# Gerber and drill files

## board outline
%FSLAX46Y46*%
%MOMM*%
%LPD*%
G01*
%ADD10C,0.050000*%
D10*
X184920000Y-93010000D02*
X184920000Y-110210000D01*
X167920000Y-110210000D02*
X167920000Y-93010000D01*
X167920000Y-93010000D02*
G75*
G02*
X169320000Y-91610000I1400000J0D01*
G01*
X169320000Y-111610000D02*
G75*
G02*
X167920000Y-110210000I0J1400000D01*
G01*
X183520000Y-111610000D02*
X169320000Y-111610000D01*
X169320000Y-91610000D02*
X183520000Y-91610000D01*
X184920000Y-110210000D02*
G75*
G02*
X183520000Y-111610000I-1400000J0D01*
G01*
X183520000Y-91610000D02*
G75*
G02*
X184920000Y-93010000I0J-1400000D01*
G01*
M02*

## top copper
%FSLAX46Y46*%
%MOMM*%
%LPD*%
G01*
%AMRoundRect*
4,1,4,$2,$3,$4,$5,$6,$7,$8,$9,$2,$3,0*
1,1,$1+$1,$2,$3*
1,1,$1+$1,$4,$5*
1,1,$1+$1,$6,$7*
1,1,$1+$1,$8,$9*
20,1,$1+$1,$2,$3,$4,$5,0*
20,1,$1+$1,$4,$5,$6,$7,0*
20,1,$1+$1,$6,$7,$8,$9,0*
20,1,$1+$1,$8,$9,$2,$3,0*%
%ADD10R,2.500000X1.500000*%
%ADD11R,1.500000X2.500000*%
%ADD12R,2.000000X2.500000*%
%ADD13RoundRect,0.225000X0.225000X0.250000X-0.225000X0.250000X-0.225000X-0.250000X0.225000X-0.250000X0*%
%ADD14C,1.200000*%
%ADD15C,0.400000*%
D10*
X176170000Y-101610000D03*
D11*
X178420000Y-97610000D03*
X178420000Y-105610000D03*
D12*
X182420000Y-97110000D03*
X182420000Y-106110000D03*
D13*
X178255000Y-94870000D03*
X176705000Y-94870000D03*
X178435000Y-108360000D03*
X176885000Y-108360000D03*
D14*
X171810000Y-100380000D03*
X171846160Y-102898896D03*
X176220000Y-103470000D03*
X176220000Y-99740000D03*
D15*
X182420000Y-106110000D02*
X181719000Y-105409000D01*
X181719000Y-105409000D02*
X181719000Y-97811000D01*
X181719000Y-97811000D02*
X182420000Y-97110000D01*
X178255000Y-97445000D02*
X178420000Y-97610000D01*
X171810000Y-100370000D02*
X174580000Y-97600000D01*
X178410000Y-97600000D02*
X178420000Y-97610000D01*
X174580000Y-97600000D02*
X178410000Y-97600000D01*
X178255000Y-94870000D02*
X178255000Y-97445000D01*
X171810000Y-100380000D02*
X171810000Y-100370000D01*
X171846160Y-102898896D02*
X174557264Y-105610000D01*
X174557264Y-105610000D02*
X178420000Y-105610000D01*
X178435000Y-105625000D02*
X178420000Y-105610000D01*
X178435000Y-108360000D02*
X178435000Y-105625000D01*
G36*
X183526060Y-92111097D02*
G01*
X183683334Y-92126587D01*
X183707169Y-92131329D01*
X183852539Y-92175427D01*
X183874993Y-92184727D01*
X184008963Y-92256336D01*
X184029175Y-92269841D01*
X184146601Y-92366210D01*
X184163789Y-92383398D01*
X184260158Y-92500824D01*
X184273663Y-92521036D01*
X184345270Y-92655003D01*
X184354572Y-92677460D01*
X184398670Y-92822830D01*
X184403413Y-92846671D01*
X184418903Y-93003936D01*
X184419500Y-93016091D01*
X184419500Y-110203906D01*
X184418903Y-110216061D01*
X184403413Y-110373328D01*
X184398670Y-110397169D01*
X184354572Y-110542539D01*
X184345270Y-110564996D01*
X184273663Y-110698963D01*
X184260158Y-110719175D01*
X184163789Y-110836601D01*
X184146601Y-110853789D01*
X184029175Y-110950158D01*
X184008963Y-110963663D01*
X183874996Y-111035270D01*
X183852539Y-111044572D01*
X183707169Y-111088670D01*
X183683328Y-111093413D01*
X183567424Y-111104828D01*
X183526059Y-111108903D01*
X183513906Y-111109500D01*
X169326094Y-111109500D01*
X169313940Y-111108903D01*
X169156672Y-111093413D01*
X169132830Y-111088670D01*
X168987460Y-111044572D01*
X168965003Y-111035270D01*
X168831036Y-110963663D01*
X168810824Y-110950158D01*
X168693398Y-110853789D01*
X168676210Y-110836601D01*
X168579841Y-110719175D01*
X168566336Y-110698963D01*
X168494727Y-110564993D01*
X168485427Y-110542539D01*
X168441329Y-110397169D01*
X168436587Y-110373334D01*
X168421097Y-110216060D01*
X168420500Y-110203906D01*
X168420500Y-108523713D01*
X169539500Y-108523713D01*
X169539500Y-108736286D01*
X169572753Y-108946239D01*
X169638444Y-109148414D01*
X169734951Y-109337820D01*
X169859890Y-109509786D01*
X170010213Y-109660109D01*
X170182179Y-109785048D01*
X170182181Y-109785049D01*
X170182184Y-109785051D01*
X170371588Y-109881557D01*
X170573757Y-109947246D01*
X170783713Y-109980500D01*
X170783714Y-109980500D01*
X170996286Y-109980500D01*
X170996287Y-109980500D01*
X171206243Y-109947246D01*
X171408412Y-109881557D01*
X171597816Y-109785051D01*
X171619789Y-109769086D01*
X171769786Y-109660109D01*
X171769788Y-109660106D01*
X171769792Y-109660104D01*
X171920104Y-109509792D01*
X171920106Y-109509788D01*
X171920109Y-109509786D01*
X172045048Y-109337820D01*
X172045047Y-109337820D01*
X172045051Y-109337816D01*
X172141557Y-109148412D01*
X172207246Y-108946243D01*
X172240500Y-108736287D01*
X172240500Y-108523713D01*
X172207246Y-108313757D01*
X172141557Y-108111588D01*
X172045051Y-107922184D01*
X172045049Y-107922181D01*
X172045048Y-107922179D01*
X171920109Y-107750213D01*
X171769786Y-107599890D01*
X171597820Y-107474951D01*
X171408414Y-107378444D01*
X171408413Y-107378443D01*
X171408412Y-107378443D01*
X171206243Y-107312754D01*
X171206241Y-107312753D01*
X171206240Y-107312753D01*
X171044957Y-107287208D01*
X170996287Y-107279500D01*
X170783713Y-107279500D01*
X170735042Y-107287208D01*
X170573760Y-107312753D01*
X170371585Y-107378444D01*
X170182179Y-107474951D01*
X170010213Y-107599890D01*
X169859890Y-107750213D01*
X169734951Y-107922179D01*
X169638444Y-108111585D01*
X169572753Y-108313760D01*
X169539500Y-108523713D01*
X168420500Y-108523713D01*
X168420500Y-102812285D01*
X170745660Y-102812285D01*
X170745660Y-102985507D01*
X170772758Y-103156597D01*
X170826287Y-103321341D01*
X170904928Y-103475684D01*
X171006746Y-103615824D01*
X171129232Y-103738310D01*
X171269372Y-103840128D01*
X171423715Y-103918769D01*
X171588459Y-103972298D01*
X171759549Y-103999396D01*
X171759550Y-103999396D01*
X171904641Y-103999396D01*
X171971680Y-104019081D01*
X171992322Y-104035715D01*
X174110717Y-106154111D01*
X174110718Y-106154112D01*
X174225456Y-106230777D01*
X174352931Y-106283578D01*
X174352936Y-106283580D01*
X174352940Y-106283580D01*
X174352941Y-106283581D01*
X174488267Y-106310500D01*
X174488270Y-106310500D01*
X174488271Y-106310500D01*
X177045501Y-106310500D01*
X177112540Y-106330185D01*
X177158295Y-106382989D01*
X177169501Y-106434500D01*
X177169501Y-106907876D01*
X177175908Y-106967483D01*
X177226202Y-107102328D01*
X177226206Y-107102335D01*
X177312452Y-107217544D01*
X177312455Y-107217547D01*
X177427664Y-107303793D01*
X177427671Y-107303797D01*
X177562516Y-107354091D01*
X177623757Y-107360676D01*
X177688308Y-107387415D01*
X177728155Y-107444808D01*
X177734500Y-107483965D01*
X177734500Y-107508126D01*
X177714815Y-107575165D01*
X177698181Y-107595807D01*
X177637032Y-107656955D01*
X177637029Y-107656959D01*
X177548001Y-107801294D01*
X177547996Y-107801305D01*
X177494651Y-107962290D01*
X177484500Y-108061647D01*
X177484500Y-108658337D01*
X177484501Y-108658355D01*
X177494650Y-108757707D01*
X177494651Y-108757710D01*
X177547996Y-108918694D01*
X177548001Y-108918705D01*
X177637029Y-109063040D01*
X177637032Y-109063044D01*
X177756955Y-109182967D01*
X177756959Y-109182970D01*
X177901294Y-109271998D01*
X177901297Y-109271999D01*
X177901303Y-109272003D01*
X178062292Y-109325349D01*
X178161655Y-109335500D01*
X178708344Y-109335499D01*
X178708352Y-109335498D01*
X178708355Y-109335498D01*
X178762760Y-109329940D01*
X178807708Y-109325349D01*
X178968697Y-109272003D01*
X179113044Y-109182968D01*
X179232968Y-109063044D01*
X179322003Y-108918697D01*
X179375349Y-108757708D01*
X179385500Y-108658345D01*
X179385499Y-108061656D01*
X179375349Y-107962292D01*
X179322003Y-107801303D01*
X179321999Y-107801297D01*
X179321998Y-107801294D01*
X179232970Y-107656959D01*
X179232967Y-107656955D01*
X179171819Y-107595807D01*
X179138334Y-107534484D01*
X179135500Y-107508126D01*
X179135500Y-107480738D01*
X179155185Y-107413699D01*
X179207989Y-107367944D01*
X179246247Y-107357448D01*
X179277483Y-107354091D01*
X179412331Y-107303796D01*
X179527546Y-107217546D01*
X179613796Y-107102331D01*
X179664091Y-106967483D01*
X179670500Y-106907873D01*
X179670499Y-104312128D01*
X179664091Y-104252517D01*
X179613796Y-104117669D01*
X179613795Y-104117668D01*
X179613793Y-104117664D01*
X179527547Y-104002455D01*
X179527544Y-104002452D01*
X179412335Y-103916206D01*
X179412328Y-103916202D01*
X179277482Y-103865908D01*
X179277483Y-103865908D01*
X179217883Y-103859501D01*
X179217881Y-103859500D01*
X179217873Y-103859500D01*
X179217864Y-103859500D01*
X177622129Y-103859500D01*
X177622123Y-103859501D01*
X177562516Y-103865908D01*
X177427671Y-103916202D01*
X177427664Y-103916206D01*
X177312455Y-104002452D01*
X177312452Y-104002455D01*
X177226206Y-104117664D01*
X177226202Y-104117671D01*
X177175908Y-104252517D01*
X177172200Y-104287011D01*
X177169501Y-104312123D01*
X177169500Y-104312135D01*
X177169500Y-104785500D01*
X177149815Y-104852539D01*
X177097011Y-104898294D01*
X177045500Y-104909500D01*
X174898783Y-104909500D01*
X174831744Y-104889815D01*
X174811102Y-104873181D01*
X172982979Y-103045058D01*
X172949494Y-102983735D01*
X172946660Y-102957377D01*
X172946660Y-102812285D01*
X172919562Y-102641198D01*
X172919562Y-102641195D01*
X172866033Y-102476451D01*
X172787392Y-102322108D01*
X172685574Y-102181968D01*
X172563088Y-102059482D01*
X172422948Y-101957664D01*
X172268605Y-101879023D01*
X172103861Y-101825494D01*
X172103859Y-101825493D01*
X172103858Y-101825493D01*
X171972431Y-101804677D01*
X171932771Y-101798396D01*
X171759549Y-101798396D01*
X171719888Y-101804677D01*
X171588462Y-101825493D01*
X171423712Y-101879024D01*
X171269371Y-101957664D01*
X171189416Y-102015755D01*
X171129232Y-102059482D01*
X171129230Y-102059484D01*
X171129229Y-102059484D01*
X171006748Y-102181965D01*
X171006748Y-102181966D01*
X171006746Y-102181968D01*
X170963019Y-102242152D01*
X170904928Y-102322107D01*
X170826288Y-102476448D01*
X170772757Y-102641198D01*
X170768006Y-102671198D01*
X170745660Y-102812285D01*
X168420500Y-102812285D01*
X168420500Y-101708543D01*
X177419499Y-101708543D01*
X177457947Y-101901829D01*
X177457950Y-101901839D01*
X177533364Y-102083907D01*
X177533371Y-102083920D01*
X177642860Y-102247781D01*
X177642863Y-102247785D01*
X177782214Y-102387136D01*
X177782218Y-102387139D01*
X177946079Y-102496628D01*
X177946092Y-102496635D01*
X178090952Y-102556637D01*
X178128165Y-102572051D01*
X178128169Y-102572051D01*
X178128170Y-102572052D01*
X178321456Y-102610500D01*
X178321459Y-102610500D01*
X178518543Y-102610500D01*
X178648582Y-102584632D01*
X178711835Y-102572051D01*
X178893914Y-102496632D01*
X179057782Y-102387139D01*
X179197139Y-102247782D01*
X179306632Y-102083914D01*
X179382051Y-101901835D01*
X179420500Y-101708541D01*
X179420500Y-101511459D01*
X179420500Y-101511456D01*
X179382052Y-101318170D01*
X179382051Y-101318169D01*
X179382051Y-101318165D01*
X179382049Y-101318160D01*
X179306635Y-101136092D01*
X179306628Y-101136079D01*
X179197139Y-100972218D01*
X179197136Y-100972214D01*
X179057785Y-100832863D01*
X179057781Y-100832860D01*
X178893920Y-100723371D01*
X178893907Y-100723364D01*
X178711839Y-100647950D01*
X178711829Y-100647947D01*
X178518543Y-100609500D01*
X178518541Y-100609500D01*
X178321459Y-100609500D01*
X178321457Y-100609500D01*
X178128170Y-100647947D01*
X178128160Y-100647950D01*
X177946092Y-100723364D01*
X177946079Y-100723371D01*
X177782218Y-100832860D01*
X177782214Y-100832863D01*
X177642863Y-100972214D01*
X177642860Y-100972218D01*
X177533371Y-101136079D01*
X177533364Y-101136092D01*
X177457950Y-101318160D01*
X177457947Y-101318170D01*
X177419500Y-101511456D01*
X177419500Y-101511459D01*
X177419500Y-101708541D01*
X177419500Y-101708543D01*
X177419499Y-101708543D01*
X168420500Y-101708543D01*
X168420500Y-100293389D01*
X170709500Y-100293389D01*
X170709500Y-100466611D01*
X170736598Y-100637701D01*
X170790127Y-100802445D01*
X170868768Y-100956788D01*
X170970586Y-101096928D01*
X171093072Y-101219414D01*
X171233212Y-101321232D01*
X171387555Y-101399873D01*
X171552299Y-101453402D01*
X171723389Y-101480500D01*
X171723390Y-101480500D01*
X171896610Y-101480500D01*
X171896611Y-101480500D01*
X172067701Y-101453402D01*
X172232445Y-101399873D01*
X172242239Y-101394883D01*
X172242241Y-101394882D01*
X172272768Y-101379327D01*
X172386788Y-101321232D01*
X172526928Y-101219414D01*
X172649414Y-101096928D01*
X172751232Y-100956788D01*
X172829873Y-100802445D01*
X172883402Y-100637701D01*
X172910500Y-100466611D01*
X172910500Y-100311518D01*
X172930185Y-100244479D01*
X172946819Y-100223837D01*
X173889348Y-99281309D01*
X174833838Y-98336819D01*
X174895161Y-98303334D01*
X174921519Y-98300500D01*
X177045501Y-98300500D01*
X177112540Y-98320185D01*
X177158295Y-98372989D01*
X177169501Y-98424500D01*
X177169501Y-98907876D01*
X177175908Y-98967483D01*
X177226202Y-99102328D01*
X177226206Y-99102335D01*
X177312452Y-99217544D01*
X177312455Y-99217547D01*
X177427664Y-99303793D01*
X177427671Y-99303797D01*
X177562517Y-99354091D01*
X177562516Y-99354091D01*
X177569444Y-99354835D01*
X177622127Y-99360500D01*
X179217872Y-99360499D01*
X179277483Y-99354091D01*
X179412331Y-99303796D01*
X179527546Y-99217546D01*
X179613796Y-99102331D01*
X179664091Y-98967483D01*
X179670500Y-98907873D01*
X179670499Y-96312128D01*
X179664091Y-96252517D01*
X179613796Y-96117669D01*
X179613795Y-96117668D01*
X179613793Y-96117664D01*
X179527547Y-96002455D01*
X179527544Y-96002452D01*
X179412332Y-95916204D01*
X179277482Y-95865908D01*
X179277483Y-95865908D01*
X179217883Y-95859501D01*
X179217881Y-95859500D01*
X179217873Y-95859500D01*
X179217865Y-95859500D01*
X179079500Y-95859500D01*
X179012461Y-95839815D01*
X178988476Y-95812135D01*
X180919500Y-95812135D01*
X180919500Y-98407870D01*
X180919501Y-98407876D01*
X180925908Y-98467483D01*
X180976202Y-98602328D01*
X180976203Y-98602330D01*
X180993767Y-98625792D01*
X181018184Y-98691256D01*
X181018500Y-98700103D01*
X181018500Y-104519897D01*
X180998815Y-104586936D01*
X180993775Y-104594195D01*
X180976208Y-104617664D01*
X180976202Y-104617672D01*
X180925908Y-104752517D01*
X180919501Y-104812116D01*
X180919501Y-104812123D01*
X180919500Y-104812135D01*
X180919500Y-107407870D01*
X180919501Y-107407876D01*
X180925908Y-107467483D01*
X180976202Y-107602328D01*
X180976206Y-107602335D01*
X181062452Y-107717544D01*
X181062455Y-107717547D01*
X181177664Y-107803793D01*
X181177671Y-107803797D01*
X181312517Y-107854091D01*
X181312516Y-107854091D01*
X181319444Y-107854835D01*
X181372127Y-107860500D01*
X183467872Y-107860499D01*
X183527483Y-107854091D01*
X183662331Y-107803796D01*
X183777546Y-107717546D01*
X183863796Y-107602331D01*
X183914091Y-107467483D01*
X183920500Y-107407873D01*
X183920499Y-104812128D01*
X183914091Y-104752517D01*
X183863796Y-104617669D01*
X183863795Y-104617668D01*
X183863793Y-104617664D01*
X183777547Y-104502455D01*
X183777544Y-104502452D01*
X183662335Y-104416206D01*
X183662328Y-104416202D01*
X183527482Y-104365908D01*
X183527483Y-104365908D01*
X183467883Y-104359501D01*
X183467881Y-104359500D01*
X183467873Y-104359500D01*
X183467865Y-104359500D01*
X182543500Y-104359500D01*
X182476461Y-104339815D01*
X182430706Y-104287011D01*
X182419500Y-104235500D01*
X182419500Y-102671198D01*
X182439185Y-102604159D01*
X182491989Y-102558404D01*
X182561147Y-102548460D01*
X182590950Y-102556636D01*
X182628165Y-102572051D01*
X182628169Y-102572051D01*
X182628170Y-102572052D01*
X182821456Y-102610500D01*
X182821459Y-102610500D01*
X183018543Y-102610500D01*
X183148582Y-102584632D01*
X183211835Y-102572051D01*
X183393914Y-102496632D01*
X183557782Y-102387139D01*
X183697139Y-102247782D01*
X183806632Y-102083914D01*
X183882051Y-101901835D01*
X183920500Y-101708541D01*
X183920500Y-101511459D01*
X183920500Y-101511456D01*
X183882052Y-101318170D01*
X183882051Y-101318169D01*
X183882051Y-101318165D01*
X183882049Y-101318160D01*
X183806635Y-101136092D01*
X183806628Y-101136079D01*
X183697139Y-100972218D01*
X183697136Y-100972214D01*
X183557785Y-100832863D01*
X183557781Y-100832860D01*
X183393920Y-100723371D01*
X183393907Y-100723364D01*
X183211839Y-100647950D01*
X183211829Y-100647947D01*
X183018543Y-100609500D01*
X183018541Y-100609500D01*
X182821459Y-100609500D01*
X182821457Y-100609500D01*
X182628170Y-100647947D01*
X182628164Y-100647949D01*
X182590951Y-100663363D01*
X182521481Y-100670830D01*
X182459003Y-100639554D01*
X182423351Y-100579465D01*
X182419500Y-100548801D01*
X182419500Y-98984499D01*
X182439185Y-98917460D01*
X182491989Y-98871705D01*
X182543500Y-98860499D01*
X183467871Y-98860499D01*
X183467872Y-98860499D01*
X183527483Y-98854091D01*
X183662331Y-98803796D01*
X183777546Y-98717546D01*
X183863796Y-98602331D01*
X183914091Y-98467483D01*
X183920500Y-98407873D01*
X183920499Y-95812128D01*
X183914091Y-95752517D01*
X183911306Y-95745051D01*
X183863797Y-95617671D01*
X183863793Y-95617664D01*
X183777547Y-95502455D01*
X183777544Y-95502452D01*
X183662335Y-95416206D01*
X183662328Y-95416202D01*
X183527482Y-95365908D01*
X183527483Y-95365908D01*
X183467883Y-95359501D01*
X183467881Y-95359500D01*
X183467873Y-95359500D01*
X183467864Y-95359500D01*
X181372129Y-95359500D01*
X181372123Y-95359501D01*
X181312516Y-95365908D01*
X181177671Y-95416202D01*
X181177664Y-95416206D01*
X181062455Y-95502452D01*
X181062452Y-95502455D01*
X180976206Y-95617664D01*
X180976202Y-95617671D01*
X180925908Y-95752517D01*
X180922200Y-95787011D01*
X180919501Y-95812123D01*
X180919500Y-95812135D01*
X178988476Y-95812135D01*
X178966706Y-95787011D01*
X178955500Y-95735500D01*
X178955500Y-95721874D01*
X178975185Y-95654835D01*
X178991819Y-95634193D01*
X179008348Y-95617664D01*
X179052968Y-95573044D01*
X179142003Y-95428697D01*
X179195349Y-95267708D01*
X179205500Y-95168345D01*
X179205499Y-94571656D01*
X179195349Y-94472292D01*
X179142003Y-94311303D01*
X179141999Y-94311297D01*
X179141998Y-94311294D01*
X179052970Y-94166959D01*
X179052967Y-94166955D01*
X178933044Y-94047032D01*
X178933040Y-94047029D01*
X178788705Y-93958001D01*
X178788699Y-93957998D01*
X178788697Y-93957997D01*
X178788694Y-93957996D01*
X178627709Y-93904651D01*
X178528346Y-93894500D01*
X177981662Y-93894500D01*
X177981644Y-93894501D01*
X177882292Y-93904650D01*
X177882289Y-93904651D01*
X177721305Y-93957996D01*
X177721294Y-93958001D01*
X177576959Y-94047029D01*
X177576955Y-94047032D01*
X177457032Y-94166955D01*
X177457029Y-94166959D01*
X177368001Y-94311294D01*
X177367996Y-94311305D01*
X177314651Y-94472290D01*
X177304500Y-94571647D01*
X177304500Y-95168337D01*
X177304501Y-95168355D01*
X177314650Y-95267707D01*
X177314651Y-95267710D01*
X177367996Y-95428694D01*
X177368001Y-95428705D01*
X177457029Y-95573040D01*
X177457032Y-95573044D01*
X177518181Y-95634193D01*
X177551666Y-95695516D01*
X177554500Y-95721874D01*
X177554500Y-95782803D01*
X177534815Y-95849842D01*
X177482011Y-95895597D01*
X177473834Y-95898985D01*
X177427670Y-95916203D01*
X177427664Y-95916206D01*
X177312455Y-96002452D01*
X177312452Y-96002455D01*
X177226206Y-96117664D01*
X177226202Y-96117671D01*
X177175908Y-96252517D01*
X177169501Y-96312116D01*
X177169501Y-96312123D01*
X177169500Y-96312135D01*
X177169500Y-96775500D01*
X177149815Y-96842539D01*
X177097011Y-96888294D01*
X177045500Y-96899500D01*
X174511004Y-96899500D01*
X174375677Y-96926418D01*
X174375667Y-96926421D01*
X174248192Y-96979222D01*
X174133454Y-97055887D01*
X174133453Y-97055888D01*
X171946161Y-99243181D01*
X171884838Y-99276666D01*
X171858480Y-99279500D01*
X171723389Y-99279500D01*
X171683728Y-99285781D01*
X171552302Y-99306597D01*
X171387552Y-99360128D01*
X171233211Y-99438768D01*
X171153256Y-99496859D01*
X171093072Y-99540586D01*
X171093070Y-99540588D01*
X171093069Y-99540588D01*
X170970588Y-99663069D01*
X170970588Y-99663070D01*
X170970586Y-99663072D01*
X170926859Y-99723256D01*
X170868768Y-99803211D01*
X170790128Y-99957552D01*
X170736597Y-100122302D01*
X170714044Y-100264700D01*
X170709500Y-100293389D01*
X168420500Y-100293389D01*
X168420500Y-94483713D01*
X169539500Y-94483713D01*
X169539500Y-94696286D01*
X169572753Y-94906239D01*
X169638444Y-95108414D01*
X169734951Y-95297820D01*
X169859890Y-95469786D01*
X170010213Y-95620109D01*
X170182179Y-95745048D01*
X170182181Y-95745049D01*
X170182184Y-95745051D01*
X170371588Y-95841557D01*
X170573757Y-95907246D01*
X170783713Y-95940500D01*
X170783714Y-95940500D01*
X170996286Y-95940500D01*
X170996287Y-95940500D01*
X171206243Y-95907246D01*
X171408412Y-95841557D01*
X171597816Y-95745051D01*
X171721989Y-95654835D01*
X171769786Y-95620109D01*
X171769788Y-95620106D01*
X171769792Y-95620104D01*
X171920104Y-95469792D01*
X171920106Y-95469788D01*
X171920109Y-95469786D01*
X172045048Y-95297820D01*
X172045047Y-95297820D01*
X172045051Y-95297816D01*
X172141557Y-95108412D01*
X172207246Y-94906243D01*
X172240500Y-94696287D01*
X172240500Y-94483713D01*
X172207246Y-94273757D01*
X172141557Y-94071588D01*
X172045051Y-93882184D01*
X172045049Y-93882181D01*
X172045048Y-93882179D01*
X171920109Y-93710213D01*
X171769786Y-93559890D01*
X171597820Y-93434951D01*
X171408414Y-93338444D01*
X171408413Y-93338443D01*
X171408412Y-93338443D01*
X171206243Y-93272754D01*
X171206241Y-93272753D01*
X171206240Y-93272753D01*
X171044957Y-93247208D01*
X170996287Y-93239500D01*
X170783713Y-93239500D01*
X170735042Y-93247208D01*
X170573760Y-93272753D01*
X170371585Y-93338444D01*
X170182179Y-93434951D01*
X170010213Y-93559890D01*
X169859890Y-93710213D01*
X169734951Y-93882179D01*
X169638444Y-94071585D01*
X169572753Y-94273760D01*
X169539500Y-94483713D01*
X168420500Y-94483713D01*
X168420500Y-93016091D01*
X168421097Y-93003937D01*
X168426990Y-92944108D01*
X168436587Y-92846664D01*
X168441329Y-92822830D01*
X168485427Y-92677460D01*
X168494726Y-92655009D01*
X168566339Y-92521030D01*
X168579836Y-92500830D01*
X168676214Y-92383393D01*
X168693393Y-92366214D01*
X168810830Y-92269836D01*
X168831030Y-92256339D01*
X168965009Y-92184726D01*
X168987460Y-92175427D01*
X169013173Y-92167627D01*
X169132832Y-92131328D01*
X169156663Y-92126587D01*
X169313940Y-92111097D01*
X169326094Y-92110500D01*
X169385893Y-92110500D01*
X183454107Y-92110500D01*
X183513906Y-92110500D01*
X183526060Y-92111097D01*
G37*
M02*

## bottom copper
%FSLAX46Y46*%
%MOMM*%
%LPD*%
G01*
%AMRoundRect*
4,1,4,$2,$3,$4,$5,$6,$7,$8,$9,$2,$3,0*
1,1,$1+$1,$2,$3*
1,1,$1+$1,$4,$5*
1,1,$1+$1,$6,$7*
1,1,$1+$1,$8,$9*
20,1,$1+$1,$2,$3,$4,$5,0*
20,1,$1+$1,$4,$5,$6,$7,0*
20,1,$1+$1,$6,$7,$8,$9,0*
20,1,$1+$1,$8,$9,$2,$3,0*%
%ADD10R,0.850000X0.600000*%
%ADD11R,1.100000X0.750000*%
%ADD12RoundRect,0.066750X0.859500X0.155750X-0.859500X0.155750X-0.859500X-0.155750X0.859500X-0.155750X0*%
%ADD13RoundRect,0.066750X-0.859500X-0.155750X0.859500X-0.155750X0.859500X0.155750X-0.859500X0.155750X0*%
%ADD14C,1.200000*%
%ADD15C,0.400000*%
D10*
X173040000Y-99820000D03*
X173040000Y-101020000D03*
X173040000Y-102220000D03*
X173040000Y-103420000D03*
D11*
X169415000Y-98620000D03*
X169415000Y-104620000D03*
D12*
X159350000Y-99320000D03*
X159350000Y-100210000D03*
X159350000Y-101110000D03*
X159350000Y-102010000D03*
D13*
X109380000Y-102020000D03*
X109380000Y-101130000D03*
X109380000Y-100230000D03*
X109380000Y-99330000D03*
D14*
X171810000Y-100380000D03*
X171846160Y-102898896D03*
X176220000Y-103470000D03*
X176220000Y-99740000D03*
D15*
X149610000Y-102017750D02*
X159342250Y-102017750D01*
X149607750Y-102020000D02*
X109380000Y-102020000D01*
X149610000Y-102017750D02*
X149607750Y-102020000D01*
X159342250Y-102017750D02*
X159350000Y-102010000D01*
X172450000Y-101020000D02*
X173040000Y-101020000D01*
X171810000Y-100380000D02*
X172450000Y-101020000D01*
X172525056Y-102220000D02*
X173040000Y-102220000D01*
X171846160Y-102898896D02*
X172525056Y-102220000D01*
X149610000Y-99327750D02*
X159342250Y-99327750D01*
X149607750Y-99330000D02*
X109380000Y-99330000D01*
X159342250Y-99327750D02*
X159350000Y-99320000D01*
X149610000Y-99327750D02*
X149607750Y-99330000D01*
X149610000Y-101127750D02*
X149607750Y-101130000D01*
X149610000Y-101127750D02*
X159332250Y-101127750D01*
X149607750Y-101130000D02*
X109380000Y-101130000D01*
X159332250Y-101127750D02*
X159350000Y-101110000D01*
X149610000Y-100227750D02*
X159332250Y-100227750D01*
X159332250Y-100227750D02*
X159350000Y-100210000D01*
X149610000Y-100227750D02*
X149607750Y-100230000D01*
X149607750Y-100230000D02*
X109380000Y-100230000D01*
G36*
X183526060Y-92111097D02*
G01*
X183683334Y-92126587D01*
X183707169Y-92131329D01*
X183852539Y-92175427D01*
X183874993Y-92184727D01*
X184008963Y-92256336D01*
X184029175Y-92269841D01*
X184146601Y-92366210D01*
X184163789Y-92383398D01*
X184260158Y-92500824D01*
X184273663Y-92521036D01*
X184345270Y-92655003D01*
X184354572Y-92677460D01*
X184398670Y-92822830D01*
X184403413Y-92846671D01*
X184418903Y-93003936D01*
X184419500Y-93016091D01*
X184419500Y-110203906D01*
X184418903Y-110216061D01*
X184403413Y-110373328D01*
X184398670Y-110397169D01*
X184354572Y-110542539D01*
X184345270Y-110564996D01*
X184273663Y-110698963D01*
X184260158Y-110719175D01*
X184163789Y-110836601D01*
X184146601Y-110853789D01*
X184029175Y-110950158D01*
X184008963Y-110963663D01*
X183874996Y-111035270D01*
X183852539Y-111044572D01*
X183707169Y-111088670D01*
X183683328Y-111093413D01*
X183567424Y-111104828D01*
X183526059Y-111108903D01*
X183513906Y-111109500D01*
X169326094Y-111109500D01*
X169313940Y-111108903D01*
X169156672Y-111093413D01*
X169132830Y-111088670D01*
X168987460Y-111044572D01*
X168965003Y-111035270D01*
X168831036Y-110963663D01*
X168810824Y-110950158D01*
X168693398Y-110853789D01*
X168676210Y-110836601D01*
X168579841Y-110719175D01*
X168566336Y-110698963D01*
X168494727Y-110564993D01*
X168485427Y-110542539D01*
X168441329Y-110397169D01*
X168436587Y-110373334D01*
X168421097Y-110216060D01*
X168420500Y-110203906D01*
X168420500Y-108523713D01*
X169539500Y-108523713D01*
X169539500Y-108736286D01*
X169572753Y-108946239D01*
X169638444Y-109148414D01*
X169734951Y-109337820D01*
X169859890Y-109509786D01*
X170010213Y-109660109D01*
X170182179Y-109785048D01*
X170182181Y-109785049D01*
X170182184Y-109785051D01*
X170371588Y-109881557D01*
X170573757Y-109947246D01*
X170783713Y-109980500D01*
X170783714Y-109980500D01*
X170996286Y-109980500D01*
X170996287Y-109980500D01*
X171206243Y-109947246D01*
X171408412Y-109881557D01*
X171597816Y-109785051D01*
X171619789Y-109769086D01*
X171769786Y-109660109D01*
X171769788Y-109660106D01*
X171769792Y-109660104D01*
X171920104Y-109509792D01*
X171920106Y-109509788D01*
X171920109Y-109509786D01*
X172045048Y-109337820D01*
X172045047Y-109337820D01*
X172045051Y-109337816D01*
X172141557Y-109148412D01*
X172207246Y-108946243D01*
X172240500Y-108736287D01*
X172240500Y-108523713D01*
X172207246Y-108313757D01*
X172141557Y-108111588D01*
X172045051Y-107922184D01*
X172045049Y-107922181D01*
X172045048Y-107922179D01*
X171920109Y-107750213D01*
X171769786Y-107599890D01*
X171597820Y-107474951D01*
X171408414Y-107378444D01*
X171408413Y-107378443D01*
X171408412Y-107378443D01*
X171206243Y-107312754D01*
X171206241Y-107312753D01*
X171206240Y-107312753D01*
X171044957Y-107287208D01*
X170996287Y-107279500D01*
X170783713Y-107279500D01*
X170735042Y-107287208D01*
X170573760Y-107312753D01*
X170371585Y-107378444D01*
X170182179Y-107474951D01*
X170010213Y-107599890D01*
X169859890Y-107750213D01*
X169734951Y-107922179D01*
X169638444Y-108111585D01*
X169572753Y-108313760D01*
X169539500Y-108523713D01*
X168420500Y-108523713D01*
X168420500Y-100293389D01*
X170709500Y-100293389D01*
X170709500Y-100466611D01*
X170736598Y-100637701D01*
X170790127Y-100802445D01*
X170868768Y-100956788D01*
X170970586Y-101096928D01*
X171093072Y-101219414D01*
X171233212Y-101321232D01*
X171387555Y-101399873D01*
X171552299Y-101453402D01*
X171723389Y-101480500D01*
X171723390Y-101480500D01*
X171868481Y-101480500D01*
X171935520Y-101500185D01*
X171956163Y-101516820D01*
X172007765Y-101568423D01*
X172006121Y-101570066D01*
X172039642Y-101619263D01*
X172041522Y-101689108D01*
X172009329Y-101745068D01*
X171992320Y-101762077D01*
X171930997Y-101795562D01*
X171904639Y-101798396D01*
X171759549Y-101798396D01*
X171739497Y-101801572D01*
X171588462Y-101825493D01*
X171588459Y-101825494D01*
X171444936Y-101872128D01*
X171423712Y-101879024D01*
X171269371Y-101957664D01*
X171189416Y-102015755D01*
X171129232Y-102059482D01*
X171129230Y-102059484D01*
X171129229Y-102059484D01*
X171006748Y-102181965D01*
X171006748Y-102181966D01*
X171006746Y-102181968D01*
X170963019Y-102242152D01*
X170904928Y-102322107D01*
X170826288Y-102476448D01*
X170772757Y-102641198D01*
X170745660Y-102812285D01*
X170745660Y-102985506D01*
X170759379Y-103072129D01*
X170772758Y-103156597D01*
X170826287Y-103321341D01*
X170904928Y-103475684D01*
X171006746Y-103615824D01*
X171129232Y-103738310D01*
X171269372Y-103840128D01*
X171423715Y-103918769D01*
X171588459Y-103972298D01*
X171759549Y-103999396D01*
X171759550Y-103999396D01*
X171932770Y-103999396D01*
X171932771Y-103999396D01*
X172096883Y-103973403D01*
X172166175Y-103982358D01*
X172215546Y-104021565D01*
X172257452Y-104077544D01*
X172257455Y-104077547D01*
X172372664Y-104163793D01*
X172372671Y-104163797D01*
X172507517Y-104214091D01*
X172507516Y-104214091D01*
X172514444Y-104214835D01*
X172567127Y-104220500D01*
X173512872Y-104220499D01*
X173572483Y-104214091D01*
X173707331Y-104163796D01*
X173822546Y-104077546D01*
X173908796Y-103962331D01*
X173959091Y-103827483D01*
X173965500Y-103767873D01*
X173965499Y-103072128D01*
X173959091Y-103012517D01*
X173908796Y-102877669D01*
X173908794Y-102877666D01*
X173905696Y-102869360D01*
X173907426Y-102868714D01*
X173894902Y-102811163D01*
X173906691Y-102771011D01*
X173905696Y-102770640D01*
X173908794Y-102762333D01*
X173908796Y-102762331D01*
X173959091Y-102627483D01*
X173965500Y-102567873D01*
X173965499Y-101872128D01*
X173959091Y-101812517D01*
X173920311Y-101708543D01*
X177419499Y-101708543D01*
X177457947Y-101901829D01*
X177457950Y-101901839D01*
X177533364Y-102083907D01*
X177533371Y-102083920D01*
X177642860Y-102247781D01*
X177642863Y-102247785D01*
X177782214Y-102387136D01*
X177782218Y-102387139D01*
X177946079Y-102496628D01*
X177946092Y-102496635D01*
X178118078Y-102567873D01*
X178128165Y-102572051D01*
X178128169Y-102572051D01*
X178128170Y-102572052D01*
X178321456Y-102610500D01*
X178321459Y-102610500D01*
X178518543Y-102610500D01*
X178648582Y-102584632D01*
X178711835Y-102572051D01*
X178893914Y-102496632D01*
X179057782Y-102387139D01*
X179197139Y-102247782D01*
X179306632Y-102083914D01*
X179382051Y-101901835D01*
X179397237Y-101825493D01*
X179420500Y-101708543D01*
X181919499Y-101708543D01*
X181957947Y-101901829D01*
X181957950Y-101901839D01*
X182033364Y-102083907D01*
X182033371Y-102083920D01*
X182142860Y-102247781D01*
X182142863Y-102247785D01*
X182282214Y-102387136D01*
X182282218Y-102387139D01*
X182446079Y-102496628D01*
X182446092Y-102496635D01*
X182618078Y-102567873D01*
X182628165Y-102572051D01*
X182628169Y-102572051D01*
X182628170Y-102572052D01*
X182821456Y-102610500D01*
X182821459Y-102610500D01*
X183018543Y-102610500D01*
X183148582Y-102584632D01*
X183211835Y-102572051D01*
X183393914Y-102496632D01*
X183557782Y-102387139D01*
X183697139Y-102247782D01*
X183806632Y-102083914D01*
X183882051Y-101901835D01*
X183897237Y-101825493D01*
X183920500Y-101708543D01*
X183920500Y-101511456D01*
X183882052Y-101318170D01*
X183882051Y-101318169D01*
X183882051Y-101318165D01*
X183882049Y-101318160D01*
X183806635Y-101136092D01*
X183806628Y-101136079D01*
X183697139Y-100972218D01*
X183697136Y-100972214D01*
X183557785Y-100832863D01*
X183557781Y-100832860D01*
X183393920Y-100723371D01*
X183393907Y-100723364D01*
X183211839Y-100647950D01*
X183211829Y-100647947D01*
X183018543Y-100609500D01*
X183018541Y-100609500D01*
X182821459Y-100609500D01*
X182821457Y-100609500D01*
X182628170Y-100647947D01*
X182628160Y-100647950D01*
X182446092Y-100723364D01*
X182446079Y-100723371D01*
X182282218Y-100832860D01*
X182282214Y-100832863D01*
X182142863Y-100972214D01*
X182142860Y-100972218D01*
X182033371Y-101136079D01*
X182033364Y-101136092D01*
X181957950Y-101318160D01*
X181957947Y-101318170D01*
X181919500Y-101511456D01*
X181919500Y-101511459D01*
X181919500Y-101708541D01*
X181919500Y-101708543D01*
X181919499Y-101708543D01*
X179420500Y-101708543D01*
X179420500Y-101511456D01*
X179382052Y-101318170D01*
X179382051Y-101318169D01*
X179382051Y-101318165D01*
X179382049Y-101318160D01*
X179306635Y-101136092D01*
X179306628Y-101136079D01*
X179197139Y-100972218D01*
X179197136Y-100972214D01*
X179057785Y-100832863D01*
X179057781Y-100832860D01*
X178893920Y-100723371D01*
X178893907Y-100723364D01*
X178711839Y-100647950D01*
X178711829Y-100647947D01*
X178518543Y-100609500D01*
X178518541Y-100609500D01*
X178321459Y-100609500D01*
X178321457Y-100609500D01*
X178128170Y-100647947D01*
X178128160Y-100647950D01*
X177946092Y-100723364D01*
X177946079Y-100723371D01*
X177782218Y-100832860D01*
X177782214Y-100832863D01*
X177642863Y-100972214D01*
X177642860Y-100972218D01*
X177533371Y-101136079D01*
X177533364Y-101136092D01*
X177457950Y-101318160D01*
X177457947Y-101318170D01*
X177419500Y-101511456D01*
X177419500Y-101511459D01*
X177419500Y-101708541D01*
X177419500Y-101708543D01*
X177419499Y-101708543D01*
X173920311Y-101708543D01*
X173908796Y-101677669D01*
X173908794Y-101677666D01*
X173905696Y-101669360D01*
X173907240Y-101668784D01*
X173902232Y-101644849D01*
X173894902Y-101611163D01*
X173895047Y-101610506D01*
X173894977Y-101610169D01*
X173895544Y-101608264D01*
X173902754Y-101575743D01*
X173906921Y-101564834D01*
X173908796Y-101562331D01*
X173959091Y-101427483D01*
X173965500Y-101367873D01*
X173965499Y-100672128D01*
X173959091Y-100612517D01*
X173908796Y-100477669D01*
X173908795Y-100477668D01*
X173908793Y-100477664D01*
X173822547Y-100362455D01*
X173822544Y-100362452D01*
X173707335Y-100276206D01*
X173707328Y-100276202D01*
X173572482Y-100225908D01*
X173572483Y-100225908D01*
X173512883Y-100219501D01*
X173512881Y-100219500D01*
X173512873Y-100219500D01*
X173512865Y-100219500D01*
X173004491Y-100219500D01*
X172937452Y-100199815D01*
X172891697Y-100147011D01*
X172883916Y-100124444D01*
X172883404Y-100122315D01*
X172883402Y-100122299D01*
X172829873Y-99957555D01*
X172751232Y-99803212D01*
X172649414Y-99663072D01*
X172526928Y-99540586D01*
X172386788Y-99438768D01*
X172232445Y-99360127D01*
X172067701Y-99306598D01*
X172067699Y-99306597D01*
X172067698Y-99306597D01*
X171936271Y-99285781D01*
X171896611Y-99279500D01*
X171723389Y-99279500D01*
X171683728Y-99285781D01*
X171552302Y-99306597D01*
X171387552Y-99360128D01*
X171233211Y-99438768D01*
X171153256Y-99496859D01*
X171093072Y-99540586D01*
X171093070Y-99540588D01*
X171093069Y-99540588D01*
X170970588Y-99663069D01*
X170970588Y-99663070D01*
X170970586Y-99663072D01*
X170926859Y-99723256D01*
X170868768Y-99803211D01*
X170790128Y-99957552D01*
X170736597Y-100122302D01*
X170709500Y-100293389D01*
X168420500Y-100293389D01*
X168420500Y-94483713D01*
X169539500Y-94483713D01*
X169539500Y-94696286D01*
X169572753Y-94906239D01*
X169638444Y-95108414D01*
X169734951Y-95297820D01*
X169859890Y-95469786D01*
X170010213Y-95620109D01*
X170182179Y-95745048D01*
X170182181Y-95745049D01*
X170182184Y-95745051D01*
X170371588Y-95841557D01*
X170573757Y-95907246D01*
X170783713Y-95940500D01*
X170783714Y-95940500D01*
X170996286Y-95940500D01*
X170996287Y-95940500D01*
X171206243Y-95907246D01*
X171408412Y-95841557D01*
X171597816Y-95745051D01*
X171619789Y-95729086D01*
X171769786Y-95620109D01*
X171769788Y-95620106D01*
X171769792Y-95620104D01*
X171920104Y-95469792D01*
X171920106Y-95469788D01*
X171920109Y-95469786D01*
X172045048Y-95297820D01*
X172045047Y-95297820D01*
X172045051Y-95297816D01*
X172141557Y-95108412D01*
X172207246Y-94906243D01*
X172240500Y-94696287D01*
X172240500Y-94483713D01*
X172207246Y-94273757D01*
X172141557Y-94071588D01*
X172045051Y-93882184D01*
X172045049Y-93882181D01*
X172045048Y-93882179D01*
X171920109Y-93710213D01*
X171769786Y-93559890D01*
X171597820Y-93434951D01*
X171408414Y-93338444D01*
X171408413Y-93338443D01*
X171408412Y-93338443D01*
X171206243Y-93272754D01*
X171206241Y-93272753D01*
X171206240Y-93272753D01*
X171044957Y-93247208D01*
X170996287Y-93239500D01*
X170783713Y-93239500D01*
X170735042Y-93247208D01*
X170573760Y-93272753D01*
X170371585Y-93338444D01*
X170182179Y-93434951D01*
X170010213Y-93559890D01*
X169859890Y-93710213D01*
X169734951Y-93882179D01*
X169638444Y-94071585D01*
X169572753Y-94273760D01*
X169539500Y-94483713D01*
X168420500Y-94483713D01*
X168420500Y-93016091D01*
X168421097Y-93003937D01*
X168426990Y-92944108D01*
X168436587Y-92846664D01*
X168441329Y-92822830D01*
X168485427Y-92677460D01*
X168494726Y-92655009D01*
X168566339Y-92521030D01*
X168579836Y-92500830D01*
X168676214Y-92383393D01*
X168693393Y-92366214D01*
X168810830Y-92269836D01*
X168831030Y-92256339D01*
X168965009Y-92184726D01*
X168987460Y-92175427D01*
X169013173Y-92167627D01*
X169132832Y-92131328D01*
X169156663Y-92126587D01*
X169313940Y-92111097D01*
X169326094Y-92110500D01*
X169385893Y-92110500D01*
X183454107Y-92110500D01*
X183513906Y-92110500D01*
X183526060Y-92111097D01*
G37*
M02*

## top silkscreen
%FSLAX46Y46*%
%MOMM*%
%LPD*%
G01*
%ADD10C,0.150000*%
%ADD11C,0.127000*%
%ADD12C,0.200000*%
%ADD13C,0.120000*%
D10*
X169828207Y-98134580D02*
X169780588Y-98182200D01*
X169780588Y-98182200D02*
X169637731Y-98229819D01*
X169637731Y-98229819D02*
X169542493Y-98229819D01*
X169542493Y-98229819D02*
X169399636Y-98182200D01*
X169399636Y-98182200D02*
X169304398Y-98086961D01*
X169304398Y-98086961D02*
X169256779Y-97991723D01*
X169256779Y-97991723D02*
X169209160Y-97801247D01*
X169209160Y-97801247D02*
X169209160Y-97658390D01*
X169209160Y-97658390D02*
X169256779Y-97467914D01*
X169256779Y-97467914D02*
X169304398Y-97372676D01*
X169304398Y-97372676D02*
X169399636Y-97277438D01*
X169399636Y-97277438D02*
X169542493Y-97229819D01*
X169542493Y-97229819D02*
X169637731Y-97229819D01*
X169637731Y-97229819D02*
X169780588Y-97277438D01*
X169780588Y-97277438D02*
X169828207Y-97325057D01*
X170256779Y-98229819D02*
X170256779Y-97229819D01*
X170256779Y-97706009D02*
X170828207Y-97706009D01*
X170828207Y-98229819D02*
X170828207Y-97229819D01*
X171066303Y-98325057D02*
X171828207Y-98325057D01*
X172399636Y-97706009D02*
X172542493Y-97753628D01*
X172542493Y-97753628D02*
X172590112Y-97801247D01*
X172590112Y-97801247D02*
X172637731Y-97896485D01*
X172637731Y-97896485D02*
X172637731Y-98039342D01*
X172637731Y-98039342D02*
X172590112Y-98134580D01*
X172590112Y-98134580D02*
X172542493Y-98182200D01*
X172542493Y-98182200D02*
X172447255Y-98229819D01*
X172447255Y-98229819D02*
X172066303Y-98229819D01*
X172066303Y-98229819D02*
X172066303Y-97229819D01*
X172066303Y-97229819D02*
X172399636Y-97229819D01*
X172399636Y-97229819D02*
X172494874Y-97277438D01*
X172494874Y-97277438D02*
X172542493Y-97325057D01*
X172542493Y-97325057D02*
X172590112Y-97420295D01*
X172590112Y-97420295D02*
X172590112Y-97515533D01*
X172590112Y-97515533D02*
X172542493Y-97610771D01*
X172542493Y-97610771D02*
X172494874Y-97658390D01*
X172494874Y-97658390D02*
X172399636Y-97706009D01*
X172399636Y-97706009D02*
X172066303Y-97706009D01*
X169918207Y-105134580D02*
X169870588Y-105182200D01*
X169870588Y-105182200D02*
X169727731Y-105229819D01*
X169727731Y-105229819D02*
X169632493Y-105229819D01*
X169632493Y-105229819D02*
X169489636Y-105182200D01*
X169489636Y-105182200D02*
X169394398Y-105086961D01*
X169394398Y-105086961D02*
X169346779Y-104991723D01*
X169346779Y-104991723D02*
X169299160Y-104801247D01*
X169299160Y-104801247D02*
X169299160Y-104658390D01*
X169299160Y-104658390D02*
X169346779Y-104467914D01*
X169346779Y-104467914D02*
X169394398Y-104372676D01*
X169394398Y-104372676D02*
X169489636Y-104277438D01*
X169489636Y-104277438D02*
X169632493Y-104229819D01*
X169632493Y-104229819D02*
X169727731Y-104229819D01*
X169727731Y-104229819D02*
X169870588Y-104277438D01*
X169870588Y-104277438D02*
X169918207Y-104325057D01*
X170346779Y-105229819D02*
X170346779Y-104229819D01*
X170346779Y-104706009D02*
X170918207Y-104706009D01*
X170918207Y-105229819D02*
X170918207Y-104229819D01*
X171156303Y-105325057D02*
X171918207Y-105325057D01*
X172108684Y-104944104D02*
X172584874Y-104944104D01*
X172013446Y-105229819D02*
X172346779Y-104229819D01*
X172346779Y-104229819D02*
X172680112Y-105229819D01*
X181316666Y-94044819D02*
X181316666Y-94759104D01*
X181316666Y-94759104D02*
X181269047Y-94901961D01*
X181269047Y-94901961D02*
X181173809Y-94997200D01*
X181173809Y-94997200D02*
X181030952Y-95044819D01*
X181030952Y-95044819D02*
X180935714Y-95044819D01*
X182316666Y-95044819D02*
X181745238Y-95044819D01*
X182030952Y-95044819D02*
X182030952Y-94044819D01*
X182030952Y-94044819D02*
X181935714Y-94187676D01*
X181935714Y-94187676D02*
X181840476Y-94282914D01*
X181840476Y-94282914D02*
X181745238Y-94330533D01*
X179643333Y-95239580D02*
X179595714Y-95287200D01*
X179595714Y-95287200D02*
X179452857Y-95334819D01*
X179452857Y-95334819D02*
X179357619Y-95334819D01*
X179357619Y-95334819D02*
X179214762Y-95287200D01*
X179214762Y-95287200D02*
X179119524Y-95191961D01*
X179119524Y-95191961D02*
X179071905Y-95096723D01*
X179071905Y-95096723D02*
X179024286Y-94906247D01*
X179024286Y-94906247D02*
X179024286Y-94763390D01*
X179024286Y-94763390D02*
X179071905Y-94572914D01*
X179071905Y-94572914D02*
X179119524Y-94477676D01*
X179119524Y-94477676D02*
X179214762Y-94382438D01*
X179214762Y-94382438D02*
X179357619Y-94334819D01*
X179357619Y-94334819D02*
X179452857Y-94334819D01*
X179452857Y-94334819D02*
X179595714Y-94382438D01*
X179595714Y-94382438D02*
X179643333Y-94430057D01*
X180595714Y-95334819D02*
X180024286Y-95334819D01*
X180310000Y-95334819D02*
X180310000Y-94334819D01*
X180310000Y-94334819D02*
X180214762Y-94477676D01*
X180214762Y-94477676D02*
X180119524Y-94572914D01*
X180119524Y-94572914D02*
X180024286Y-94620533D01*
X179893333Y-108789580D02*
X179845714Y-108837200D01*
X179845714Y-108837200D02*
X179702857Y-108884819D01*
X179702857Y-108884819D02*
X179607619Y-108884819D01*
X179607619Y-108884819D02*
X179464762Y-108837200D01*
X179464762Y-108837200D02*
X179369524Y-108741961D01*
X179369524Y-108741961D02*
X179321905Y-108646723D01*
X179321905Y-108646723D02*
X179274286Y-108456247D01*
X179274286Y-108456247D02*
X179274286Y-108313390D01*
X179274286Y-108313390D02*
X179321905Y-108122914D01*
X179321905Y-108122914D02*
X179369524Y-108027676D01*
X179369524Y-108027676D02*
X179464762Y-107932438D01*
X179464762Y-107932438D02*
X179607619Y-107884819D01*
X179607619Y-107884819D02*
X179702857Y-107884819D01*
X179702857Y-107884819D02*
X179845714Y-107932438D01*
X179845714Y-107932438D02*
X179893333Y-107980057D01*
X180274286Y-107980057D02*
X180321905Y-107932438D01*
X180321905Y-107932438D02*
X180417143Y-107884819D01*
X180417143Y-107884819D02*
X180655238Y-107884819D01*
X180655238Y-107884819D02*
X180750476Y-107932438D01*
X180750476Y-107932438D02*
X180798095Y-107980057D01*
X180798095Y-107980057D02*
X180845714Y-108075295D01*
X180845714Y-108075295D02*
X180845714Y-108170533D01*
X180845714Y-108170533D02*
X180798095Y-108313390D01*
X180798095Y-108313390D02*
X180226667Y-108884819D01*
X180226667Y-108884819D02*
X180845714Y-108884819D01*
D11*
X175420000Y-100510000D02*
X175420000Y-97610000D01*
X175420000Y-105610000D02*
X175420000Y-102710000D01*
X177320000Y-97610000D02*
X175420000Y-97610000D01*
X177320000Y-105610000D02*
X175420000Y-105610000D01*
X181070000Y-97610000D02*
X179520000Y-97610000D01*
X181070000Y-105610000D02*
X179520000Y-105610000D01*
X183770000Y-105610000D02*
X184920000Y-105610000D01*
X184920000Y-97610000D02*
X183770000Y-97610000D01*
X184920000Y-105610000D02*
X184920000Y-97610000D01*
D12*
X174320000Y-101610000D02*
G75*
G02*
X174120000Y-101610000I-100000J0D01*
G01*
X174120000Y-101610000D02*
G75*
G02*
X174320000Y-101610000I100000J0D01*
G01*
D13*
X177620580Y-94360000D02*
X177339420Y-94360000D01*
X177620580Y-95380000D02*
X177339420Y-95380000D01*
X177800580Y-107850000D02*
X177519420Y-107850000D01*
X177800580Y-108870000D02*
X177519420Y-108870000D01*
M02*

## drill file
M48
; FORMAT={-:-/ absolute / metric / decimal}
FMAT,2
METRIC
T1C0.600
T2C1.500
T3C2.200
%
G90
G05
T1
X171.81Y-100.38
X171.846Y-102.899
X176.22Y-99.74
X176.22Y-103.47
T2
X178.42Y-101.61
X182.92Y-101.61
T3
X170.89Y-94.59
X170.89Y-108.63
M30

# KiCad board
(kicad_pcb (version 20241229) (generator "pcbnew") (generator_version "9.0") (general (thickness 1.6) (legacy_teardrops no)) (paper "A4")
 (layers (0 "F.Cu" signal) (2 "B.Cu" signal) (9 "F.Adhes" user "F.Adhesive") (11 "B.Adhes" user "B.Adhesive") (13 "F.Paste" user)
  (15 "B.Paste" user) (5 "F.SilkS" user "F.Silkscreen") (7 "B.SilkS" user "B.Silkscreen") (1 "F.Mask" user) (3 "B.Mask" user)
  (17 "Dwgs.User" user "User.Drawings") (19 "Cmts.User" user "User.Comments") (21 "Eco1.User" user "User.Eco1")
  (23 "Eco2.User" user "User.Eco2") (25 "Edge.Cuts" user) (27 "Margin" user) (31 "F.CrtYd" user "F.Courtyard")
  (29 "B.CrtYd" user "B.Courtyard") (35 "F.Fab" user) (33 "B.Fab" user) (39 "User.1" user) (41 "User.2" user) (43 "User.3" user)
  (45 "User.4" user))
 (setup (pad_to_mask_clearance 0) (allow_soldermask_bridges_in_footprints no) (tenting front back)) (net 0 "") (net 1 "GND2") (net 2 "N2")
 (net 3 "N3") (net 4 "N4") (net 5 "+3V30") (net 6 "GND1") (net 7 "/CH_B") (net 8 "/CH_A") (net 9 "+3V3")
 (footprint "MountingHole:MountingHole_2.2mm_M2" (layer "F.Cu") (at 170.89 94.59)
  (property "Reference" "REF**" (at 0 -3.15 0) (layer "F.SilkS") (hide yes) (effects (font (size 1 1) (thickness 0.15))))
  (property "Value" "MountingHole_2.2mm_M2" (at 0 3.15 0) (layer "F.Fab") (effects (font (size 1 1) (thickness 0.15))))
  (pad "" np_thru_hole circle (at 0 0) (size 2.2 2.2) (drill 2.2) (layers "*.Cu" "*.Mask")))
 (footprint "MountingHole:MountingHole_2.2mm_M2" (layer "F.Cu") (at 170.89 108.63)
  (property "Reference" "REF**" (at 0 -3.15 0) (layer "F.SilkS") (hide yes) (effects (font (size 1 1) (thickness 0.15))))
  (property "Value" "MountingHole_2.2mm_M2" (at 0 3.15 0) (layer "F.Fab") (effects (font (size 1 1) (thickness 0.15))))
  (pad "" np_thru_hole circle (at 0 0) (size 2.2 2.2) (drill 2.2) (layers "*.Cu" "*.Mask")))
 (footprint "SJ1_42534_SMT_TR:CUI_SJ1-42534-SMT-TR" (layer "F.Cu") (at 180.17 101.61 180)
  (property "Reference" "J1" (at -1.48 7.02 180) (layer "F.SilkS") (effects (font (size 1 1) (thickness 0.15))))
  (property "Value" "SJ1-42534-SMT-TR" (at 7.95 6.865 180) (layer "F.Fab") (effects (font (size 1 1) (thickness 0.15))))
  (fp_line (start 4.75 1.1) (end 4.75 4) (stroke (width 0.127) (type solid)) (layer "F.SilkS"))
  (fp_line (start 4.75 -4) (end 4.75 -1.1) (stroke (width 0.127) (type solid)) (layer "F.SilkS"))
  (fp_line (start 2.85 4) (end 4.75 4) (stroke (width 0.127) (type solid)) (layer "F.SilkS"))
  (fp_line (start 2.85 -4) (end 4.75 -4) (stroke (width 0.127) (type solid)) (layer "F.SilkS"))
  (fp_line (start -0.9 4) (end 0.65 4) (stroke (width 0.127) (type solid)) (layer "F.SilkS"))
  (fp_line (start -0.9 -4) (end 0.65 -4) (stroke (width 0.127) (type solid)) (layer "F.SilkS"))
  (fp_line (start -3.6 -4) (end -4.75 -4) (stroke (width 0.127) (type solid)) (layer "F.SilkS"))
  (fp_line (start -4.75 4) (end -3.6 4) (stroke (width 0.127) (type solid)) (layer "F.SilkS"))
  (fp_line (start -4.75 -4) (end -4.75 4) (stroke (width 0.127) (type solid)) (layer "F.SilkS"))
  (fp_circle (center 5.95 0) (end 6.05 0) (stroke (width 0.2) (type solid)) (fill no) (layer "F.SilkS"))
  (pad "" np_thru_hole circle (at -2.75 0 180) (size 1.5 1.5) (drill 1.5) (layers "*.Cu" "*.Mask"))
  (pad "" np_thru_hole circle (at 1.75 0 180) (size 1.5 1.5) (drill 1.5) (layers "*.Cu" "*.Mask"))
  (pad "1" smd rect (at 4 0 180) (size 2.5 1.5) (layers "F.Cu" "F.Mask" "F.Paste") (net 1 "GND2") (solder_mask_margin 0.102))
  (pad "2" smd rect (at 1.75 4 180) (size 1.5 2.5) (layers "F.Cu" "F.Mask" "F.Paste") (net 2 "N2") (solder_mask_margin 0.102))
  (pad "3" smd rect (at 1.75 -4 180) (size 1.5 2.5) (layers "F.Cu" "F.Mask" "F.Paste") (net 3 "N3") (solder_mask_margin 0.102))
  (pad "4_1" smd rect (at -2.25 4.5 180) (size 2 2.5) (layers "F.Cu" "F.Mask" "F.Paste") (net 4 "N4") (solder_mask_margin 0.102))
  (pad "4_2" smd rect (at -2.25 -4.5 180) (size 2 2.5) (layers "F.Cu" "F.Mask" "F.Paste") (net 4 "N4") (solder_mask_margin 0.102)))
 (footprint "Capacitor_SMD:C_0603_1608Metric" (layer "F.Cu") (at 177.48 94.87 180)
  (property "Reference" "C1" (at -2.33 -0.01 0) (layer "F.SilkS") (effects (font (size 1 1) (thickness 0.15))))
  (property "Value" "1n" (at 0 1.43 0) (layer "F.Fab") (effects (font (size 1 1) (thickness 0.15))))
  (fp_line (start -0.14058 0.51) (end 0.14058 0.51) (stroke (width 0.12) (type solid)) (layer "F.SilkS"))
  (fp_line (start -0.14058 -0.51) (end 0.14058 -0.51) (stroke (width 0.12) (type solid)) (layer "F.SilkS"))
  (pad "1" smd roundrect (at -0.775 0 180) (size 0.9 0.95) (layers "F.Cu" "F.Mask" "F.Paste") (roundrect_rratio 0.25) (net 2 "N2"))
  (pad "2" smd roundrect (at 0.775 0 180) (size 0.9 0.95) (layers "F.Cu" "F.Mask" "F.Paste") (roundrect_rratio 0.25) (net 1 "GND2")))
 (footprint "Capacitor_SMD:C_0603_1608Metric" (layer "F.Cu") (at 177.66 108.36 180)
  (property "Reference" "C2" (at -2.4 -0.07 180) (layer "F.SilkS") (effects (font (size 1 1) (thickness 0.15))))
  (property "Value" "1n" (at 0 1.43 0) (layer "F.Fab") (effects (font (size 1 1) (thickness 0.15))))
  (fp_line (start -0.14058 0.51) (end 0.14058 0.51) (stroke (width 0.12) (type solid)) (layer "F.SilkS"))
  (fp_line (start -0.14058 -0.51) (end 0.14058 -0.51) (stroke (width 0.12) (type solid)) (layer "F.SilkS"))
  (pad "1" smd roundrect (at -0.775 0 180) (size 0.9 0.95) (layers "F.Cu" "F.Mask" "F.Paste") (roundrect_rratio 0.25) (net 3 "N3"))
  (pad "2" smd roundrect (at 0.775 0 180) (size 0.9 0.95) (layers "F.Cu" "F.Mask" "F.Paste") (roundrect_rratio 0.25) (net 1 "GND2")))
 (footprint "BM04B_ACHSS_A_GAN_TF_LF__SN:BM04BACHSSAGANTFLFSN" (layer "B.Cu") (at 171.375 101.64 180)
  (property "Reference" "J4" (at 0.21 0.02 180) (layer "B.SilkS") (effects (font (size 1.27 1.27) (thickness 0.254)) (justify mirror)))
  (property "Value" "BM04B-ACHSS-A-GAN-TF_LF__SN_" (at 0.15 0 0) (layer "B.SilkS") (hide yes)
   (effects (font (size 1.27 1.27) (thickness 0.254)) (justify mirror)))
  (pad "1" smd rect (at -1.665 1.82 270) (size 0.6 0.85) (layers "B.Cu" "B.Mask" "B.Paste") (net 1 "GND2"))
  (pad "2" smd rect (at -1.665 0.62 270) (size 0.6 0.85) (layers "B.Cu" "B.Mask" "B.Paste") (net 2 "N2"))
  (pad "3" smd rect (at -1.665 -0.58 270) (size 0.6 0.85) (layers "B.Cu" "B.Mask" "B.Paste") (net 3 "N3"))
  (pad "4" smd rect (at -1.665 -1.78 270) (size 0.6 0.85) (layers "B.Cu" "B.Mask" "B.Paste") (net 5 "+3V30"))
  (pad "MP1" smd rect (at 1.96 3.02 270) (size 0.75 1.1) (layers "B.Cu" "B.Mask" "B.Paste") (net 1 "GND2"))
  (pad "MP2" smd rect (at 1.96 -2.98 270) (size 0.75 1.1) (layers "B.Cu" "B.Mask" "B.Paste") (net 1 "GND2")))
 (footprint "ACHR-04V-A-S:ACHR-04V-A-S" (layer "B.Cu") (at 159.36 100.66 180)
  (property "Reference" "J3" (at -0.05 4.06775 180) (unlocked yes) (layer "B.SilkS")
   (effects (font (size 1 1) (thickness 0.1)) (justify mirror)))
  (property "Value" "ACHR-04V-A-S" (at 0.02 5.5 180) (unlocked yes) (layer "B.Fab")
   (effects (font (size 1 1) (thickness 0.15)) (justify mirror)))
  (pad "1" connect roundrect (at 0.01 1.34 180) (size 1.8525 0.445) (layers "B.Cu") (roundrect_rratio 0.15) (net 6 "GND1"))
  (pad "2" connect roundrect (at 0.01 0.45 180) (size 1.8525 0.445) (layers "B.Cu") (roundrect_rratio 0.15) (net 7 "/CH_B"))
  (pad "3" connect roundrect (at 0.01 -0.45 180) (size 1.8525 0.445) (layers "B.Cu") (roundrect_rratio 0.15) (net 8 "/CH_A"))
  (pad "4" connect roundrect (at 0.01 -1.35 180) (size 1.8525 0.445) (layers "B.Cu") (roundrect_rratio 0.15) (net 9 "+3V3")))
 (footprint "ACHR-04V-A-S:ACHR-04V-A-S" (layer "B.Cu") (at 109.37 100.68)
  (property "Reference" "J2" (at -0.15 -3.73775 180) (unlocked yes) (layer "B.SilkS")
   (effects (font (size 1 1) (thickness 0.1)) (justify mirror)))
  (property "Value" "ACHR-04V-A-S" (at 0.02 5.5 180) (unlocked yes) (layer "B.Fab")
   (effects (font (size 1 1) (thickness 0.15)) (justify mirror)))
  (pad "1" connect roundrect (at 0.01 1.34) (size 1.8525 0.445) (layers "B.Cu") (roundrect_rratio 0.15) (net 9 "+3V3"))
  (pad "2" connect roundrect (at 0.01 0.45) (size 1.8525 0.445) (layers "B.Cu") (roundrect_rratio 0.15) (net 8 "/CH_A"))
  (pad "3" connect roundrect (at 0.01 -0.45) (size 1.8525 0.445) (layers "B.Cu") (roundrect_rratio 0.15) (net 7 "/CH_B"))
  (pad "4" connect roundrect (at 0.01 -1.35) (size 1.8525 0.445) (layers "B.Cu") (roundrect_rratio 0.15) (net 6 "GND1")))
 (gr_line (start 184.92 93.01) (end 184.92 110.21) (stroke (width 0.05) (type default)) (layer "Edge.Cuts"))
 (gr_line (start 167.92 110.21) (end 167.92 93.01) (stroke (width 0.05) (type default)) (layer "Edge.Cuts"))
 (gr_arc (start 167.92 93.01) (mid 168.330051 92.020051) (end 169.32 91.61) (stroke (width 0.05) (type default)) (layer "Edge.Cuts"))
 (gr_arc (start 169.32 111.61) (mid 168.330051 111.199949) (end 167.92 110.21) (stroke (width 0.05) (type default)) (layer "Edge.Cuts"))
 (gr_line (start 183.52 111.61) (end 169.32 111.61) (stroke (width 0.05) (type default)) (layer "Edge.Cuts"))
 (gr_line (start 169.32 91.61) (end 183.52 91.61) (stroke (width 0.05) (type default)) (layer "Edge.Cuts"))
 (gr_arc (start 184.92 110.21) (mid 184.509949 111.199949) (end 183.52 111.61) (stroke (width 0.05) (type default)) (layer "Edge.Cuts"))
 (gr_arc (start 183.52 91.61) (mid 184.509949 92.020051) (end 184.92 93.01) (stroke (width 0.05) (type default)) (layer "Edge.Cuts"))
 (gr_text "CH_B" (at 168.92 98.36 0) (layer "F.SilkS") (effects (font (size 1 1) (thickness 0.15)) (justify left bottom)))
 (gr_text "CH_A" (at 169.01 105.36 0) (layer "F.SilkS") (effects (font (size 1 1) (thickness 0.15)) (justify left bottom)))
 (segment (start 149.61 102.01775) (end 159.34225 102.01775) (width 0.4) (layer "B.Cu") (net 9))
 (segment (start 149.60775 102.02) (end 109.38 102.02) (width 0.4) (layer "B.Cu") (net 9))
 (segment (start 149.61 102.01775) (end 149.60775 102.02) (width 0.4) (layer "B.Cu") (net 9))
 (segment (start 159.34225 102.01775) (end 159.35 102.01) (width 0.4) (layer "B.Cu") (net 9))
 (segment (start 182.42 106.11) (end 181.719 105.409) (width 0.4) (layer "F.Cu") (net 4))
 (segment (start 181.719 105.409) (end 181.719 97.811) (width 0.4) (layer "F.Cu") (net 4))
 (segment (start 181.719 97.811) (end 182.42 97.11) (width 0.4) (layer "F.Cu") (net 4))
 (segment (start 178.255 97.445) (end 178.42 97.61) (width 0.4) (layer "F.Cu") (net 2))
 (segment (start 171.81 100.37) (end 174.58 97.6) (width 0.4) (layer "F.Cu") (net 2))
 (segment (start 178.41 97.6) (end 178.42 97.61) (width 0.4) (layer "F.Cu") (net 2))
 (segment (start 174.58 97.6) (end 178.41 97.6) (width 0.4) (layer "F.Cu") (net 2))
 (segment (start 178.255 94.87) (end 178.255 97.445) (width 0.4) (layer "F.Cu") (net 2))
 (segment (start 171.81 100.38) (end 171.81 100.37) (width 0.4) (layer "F.Cu") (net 2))
 (via (at 171.81 100.38) (size 1.2) (drill 0.6) (layers "F.Cu" "B.Cu") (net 2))
 (segment (start 172.45 101.02) (end 173.04 101.02) (width 0.4) (layer "B.Cu") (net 2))
 (segment (start 171.81 100.38) (end 172.45 101.02) (width 0.4) (layer "B.Cu") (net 2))
 (segment (start 171.84616 102.898896) (end 174.557264 105.61) (width 0.4) (layer "F.Cu") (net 3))
 (segment (start 174.557264 105.61) (end 178.42 105.61) (width 0.4) (layer "F.Cu") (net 3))
 (segment (start 178.435 105.625) (end 178.42 105.61) (width 0.4) (layer "F.Cu") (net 3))
 (segment (start 178.435 108.36) (end 178.435 105.625) (width 0.4) (layer "F.Cu") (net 3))
 (via (at 171.84616 102.898896) (size 1.2) (drill 0.6) (layers "F.Cu" "B.Cu") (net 3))
 (segment (start 172.525056 102.22) (end 173.04 102.22) (width 0.4) (layer "B.Cu") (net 3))
 (segment (start 171.84616 102.898896) (end 172.525056 102.22) (width 0.4) (layer "B.Cu") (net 3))
 (via (at 176.22 103.47) (size 1.2) (drill 0.6) (layers "F.Cu" "B.Cu") (free yes) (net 1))
 (via (at 176.22 99.74) (size 1.2) (drill 0.6) (layers "F.Cu" "B.Cu") (free yes) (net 1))
 (segment (start 149.61 99.32775) (end 159.34225 99.32775) (width 0.4) (layer "B.Cu") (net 6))
 (segment (start 149.60775 99.33) (end 109.38 99.33) (width 0.4) (layer "B.Cu") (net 6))
 (segment (start 159.34225 99.32775) (end 159.35 99.32) (width 0.4) (layer "B.Cu") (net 6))
 (segment (start 149.61 99.32775) (end 149.60775 99.33) (width 0.4) (layer "B.Cu") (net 6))
 (segment (start 149.61 101.12775) (end 149.60775 101.13) (width 0.4) (layer "B.Cu") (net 8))
 (segment (start 149.61 101.12775) (end 159.33225 101.12775) (width 0.4) (layer "B.Cu") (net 8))
 (segment (start 149.60775 101.13) (end 109.38 101.13) (width 0.4) (layer "B.Cu") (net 8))
 (segment (start 159.33225 101.12775) (end 159.35 101.11) (width 0.4) (layer "B.Cu") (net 8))
 (segment (start 149.61 100.22775) (end 159.33225 100.22775) (width 0.4) (layer "B.Cu") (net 7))
 (segment (start 159.33225 100.22775) (end 159.35 100.21) (width 0.4) (layer "B.Cu") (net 7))
 (segment (start 149.61 100.22775) (end 149.60775 100.23) (width 0.4) (layer "B.Cu") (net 7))
 (segment (start 149.60775 100.23) (end 109.38 100.23) (width 0.4) (layer "B.Cu") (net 7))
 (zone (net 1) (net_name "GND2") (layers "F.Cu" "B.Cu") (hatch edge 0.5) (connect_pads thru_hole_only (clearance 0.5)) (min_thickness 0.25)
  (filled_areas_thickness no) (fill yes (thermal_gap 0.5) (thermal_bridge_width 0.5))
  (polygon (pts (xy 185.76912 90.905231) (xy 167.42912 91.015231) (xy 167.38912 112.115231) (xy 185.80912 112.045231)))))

